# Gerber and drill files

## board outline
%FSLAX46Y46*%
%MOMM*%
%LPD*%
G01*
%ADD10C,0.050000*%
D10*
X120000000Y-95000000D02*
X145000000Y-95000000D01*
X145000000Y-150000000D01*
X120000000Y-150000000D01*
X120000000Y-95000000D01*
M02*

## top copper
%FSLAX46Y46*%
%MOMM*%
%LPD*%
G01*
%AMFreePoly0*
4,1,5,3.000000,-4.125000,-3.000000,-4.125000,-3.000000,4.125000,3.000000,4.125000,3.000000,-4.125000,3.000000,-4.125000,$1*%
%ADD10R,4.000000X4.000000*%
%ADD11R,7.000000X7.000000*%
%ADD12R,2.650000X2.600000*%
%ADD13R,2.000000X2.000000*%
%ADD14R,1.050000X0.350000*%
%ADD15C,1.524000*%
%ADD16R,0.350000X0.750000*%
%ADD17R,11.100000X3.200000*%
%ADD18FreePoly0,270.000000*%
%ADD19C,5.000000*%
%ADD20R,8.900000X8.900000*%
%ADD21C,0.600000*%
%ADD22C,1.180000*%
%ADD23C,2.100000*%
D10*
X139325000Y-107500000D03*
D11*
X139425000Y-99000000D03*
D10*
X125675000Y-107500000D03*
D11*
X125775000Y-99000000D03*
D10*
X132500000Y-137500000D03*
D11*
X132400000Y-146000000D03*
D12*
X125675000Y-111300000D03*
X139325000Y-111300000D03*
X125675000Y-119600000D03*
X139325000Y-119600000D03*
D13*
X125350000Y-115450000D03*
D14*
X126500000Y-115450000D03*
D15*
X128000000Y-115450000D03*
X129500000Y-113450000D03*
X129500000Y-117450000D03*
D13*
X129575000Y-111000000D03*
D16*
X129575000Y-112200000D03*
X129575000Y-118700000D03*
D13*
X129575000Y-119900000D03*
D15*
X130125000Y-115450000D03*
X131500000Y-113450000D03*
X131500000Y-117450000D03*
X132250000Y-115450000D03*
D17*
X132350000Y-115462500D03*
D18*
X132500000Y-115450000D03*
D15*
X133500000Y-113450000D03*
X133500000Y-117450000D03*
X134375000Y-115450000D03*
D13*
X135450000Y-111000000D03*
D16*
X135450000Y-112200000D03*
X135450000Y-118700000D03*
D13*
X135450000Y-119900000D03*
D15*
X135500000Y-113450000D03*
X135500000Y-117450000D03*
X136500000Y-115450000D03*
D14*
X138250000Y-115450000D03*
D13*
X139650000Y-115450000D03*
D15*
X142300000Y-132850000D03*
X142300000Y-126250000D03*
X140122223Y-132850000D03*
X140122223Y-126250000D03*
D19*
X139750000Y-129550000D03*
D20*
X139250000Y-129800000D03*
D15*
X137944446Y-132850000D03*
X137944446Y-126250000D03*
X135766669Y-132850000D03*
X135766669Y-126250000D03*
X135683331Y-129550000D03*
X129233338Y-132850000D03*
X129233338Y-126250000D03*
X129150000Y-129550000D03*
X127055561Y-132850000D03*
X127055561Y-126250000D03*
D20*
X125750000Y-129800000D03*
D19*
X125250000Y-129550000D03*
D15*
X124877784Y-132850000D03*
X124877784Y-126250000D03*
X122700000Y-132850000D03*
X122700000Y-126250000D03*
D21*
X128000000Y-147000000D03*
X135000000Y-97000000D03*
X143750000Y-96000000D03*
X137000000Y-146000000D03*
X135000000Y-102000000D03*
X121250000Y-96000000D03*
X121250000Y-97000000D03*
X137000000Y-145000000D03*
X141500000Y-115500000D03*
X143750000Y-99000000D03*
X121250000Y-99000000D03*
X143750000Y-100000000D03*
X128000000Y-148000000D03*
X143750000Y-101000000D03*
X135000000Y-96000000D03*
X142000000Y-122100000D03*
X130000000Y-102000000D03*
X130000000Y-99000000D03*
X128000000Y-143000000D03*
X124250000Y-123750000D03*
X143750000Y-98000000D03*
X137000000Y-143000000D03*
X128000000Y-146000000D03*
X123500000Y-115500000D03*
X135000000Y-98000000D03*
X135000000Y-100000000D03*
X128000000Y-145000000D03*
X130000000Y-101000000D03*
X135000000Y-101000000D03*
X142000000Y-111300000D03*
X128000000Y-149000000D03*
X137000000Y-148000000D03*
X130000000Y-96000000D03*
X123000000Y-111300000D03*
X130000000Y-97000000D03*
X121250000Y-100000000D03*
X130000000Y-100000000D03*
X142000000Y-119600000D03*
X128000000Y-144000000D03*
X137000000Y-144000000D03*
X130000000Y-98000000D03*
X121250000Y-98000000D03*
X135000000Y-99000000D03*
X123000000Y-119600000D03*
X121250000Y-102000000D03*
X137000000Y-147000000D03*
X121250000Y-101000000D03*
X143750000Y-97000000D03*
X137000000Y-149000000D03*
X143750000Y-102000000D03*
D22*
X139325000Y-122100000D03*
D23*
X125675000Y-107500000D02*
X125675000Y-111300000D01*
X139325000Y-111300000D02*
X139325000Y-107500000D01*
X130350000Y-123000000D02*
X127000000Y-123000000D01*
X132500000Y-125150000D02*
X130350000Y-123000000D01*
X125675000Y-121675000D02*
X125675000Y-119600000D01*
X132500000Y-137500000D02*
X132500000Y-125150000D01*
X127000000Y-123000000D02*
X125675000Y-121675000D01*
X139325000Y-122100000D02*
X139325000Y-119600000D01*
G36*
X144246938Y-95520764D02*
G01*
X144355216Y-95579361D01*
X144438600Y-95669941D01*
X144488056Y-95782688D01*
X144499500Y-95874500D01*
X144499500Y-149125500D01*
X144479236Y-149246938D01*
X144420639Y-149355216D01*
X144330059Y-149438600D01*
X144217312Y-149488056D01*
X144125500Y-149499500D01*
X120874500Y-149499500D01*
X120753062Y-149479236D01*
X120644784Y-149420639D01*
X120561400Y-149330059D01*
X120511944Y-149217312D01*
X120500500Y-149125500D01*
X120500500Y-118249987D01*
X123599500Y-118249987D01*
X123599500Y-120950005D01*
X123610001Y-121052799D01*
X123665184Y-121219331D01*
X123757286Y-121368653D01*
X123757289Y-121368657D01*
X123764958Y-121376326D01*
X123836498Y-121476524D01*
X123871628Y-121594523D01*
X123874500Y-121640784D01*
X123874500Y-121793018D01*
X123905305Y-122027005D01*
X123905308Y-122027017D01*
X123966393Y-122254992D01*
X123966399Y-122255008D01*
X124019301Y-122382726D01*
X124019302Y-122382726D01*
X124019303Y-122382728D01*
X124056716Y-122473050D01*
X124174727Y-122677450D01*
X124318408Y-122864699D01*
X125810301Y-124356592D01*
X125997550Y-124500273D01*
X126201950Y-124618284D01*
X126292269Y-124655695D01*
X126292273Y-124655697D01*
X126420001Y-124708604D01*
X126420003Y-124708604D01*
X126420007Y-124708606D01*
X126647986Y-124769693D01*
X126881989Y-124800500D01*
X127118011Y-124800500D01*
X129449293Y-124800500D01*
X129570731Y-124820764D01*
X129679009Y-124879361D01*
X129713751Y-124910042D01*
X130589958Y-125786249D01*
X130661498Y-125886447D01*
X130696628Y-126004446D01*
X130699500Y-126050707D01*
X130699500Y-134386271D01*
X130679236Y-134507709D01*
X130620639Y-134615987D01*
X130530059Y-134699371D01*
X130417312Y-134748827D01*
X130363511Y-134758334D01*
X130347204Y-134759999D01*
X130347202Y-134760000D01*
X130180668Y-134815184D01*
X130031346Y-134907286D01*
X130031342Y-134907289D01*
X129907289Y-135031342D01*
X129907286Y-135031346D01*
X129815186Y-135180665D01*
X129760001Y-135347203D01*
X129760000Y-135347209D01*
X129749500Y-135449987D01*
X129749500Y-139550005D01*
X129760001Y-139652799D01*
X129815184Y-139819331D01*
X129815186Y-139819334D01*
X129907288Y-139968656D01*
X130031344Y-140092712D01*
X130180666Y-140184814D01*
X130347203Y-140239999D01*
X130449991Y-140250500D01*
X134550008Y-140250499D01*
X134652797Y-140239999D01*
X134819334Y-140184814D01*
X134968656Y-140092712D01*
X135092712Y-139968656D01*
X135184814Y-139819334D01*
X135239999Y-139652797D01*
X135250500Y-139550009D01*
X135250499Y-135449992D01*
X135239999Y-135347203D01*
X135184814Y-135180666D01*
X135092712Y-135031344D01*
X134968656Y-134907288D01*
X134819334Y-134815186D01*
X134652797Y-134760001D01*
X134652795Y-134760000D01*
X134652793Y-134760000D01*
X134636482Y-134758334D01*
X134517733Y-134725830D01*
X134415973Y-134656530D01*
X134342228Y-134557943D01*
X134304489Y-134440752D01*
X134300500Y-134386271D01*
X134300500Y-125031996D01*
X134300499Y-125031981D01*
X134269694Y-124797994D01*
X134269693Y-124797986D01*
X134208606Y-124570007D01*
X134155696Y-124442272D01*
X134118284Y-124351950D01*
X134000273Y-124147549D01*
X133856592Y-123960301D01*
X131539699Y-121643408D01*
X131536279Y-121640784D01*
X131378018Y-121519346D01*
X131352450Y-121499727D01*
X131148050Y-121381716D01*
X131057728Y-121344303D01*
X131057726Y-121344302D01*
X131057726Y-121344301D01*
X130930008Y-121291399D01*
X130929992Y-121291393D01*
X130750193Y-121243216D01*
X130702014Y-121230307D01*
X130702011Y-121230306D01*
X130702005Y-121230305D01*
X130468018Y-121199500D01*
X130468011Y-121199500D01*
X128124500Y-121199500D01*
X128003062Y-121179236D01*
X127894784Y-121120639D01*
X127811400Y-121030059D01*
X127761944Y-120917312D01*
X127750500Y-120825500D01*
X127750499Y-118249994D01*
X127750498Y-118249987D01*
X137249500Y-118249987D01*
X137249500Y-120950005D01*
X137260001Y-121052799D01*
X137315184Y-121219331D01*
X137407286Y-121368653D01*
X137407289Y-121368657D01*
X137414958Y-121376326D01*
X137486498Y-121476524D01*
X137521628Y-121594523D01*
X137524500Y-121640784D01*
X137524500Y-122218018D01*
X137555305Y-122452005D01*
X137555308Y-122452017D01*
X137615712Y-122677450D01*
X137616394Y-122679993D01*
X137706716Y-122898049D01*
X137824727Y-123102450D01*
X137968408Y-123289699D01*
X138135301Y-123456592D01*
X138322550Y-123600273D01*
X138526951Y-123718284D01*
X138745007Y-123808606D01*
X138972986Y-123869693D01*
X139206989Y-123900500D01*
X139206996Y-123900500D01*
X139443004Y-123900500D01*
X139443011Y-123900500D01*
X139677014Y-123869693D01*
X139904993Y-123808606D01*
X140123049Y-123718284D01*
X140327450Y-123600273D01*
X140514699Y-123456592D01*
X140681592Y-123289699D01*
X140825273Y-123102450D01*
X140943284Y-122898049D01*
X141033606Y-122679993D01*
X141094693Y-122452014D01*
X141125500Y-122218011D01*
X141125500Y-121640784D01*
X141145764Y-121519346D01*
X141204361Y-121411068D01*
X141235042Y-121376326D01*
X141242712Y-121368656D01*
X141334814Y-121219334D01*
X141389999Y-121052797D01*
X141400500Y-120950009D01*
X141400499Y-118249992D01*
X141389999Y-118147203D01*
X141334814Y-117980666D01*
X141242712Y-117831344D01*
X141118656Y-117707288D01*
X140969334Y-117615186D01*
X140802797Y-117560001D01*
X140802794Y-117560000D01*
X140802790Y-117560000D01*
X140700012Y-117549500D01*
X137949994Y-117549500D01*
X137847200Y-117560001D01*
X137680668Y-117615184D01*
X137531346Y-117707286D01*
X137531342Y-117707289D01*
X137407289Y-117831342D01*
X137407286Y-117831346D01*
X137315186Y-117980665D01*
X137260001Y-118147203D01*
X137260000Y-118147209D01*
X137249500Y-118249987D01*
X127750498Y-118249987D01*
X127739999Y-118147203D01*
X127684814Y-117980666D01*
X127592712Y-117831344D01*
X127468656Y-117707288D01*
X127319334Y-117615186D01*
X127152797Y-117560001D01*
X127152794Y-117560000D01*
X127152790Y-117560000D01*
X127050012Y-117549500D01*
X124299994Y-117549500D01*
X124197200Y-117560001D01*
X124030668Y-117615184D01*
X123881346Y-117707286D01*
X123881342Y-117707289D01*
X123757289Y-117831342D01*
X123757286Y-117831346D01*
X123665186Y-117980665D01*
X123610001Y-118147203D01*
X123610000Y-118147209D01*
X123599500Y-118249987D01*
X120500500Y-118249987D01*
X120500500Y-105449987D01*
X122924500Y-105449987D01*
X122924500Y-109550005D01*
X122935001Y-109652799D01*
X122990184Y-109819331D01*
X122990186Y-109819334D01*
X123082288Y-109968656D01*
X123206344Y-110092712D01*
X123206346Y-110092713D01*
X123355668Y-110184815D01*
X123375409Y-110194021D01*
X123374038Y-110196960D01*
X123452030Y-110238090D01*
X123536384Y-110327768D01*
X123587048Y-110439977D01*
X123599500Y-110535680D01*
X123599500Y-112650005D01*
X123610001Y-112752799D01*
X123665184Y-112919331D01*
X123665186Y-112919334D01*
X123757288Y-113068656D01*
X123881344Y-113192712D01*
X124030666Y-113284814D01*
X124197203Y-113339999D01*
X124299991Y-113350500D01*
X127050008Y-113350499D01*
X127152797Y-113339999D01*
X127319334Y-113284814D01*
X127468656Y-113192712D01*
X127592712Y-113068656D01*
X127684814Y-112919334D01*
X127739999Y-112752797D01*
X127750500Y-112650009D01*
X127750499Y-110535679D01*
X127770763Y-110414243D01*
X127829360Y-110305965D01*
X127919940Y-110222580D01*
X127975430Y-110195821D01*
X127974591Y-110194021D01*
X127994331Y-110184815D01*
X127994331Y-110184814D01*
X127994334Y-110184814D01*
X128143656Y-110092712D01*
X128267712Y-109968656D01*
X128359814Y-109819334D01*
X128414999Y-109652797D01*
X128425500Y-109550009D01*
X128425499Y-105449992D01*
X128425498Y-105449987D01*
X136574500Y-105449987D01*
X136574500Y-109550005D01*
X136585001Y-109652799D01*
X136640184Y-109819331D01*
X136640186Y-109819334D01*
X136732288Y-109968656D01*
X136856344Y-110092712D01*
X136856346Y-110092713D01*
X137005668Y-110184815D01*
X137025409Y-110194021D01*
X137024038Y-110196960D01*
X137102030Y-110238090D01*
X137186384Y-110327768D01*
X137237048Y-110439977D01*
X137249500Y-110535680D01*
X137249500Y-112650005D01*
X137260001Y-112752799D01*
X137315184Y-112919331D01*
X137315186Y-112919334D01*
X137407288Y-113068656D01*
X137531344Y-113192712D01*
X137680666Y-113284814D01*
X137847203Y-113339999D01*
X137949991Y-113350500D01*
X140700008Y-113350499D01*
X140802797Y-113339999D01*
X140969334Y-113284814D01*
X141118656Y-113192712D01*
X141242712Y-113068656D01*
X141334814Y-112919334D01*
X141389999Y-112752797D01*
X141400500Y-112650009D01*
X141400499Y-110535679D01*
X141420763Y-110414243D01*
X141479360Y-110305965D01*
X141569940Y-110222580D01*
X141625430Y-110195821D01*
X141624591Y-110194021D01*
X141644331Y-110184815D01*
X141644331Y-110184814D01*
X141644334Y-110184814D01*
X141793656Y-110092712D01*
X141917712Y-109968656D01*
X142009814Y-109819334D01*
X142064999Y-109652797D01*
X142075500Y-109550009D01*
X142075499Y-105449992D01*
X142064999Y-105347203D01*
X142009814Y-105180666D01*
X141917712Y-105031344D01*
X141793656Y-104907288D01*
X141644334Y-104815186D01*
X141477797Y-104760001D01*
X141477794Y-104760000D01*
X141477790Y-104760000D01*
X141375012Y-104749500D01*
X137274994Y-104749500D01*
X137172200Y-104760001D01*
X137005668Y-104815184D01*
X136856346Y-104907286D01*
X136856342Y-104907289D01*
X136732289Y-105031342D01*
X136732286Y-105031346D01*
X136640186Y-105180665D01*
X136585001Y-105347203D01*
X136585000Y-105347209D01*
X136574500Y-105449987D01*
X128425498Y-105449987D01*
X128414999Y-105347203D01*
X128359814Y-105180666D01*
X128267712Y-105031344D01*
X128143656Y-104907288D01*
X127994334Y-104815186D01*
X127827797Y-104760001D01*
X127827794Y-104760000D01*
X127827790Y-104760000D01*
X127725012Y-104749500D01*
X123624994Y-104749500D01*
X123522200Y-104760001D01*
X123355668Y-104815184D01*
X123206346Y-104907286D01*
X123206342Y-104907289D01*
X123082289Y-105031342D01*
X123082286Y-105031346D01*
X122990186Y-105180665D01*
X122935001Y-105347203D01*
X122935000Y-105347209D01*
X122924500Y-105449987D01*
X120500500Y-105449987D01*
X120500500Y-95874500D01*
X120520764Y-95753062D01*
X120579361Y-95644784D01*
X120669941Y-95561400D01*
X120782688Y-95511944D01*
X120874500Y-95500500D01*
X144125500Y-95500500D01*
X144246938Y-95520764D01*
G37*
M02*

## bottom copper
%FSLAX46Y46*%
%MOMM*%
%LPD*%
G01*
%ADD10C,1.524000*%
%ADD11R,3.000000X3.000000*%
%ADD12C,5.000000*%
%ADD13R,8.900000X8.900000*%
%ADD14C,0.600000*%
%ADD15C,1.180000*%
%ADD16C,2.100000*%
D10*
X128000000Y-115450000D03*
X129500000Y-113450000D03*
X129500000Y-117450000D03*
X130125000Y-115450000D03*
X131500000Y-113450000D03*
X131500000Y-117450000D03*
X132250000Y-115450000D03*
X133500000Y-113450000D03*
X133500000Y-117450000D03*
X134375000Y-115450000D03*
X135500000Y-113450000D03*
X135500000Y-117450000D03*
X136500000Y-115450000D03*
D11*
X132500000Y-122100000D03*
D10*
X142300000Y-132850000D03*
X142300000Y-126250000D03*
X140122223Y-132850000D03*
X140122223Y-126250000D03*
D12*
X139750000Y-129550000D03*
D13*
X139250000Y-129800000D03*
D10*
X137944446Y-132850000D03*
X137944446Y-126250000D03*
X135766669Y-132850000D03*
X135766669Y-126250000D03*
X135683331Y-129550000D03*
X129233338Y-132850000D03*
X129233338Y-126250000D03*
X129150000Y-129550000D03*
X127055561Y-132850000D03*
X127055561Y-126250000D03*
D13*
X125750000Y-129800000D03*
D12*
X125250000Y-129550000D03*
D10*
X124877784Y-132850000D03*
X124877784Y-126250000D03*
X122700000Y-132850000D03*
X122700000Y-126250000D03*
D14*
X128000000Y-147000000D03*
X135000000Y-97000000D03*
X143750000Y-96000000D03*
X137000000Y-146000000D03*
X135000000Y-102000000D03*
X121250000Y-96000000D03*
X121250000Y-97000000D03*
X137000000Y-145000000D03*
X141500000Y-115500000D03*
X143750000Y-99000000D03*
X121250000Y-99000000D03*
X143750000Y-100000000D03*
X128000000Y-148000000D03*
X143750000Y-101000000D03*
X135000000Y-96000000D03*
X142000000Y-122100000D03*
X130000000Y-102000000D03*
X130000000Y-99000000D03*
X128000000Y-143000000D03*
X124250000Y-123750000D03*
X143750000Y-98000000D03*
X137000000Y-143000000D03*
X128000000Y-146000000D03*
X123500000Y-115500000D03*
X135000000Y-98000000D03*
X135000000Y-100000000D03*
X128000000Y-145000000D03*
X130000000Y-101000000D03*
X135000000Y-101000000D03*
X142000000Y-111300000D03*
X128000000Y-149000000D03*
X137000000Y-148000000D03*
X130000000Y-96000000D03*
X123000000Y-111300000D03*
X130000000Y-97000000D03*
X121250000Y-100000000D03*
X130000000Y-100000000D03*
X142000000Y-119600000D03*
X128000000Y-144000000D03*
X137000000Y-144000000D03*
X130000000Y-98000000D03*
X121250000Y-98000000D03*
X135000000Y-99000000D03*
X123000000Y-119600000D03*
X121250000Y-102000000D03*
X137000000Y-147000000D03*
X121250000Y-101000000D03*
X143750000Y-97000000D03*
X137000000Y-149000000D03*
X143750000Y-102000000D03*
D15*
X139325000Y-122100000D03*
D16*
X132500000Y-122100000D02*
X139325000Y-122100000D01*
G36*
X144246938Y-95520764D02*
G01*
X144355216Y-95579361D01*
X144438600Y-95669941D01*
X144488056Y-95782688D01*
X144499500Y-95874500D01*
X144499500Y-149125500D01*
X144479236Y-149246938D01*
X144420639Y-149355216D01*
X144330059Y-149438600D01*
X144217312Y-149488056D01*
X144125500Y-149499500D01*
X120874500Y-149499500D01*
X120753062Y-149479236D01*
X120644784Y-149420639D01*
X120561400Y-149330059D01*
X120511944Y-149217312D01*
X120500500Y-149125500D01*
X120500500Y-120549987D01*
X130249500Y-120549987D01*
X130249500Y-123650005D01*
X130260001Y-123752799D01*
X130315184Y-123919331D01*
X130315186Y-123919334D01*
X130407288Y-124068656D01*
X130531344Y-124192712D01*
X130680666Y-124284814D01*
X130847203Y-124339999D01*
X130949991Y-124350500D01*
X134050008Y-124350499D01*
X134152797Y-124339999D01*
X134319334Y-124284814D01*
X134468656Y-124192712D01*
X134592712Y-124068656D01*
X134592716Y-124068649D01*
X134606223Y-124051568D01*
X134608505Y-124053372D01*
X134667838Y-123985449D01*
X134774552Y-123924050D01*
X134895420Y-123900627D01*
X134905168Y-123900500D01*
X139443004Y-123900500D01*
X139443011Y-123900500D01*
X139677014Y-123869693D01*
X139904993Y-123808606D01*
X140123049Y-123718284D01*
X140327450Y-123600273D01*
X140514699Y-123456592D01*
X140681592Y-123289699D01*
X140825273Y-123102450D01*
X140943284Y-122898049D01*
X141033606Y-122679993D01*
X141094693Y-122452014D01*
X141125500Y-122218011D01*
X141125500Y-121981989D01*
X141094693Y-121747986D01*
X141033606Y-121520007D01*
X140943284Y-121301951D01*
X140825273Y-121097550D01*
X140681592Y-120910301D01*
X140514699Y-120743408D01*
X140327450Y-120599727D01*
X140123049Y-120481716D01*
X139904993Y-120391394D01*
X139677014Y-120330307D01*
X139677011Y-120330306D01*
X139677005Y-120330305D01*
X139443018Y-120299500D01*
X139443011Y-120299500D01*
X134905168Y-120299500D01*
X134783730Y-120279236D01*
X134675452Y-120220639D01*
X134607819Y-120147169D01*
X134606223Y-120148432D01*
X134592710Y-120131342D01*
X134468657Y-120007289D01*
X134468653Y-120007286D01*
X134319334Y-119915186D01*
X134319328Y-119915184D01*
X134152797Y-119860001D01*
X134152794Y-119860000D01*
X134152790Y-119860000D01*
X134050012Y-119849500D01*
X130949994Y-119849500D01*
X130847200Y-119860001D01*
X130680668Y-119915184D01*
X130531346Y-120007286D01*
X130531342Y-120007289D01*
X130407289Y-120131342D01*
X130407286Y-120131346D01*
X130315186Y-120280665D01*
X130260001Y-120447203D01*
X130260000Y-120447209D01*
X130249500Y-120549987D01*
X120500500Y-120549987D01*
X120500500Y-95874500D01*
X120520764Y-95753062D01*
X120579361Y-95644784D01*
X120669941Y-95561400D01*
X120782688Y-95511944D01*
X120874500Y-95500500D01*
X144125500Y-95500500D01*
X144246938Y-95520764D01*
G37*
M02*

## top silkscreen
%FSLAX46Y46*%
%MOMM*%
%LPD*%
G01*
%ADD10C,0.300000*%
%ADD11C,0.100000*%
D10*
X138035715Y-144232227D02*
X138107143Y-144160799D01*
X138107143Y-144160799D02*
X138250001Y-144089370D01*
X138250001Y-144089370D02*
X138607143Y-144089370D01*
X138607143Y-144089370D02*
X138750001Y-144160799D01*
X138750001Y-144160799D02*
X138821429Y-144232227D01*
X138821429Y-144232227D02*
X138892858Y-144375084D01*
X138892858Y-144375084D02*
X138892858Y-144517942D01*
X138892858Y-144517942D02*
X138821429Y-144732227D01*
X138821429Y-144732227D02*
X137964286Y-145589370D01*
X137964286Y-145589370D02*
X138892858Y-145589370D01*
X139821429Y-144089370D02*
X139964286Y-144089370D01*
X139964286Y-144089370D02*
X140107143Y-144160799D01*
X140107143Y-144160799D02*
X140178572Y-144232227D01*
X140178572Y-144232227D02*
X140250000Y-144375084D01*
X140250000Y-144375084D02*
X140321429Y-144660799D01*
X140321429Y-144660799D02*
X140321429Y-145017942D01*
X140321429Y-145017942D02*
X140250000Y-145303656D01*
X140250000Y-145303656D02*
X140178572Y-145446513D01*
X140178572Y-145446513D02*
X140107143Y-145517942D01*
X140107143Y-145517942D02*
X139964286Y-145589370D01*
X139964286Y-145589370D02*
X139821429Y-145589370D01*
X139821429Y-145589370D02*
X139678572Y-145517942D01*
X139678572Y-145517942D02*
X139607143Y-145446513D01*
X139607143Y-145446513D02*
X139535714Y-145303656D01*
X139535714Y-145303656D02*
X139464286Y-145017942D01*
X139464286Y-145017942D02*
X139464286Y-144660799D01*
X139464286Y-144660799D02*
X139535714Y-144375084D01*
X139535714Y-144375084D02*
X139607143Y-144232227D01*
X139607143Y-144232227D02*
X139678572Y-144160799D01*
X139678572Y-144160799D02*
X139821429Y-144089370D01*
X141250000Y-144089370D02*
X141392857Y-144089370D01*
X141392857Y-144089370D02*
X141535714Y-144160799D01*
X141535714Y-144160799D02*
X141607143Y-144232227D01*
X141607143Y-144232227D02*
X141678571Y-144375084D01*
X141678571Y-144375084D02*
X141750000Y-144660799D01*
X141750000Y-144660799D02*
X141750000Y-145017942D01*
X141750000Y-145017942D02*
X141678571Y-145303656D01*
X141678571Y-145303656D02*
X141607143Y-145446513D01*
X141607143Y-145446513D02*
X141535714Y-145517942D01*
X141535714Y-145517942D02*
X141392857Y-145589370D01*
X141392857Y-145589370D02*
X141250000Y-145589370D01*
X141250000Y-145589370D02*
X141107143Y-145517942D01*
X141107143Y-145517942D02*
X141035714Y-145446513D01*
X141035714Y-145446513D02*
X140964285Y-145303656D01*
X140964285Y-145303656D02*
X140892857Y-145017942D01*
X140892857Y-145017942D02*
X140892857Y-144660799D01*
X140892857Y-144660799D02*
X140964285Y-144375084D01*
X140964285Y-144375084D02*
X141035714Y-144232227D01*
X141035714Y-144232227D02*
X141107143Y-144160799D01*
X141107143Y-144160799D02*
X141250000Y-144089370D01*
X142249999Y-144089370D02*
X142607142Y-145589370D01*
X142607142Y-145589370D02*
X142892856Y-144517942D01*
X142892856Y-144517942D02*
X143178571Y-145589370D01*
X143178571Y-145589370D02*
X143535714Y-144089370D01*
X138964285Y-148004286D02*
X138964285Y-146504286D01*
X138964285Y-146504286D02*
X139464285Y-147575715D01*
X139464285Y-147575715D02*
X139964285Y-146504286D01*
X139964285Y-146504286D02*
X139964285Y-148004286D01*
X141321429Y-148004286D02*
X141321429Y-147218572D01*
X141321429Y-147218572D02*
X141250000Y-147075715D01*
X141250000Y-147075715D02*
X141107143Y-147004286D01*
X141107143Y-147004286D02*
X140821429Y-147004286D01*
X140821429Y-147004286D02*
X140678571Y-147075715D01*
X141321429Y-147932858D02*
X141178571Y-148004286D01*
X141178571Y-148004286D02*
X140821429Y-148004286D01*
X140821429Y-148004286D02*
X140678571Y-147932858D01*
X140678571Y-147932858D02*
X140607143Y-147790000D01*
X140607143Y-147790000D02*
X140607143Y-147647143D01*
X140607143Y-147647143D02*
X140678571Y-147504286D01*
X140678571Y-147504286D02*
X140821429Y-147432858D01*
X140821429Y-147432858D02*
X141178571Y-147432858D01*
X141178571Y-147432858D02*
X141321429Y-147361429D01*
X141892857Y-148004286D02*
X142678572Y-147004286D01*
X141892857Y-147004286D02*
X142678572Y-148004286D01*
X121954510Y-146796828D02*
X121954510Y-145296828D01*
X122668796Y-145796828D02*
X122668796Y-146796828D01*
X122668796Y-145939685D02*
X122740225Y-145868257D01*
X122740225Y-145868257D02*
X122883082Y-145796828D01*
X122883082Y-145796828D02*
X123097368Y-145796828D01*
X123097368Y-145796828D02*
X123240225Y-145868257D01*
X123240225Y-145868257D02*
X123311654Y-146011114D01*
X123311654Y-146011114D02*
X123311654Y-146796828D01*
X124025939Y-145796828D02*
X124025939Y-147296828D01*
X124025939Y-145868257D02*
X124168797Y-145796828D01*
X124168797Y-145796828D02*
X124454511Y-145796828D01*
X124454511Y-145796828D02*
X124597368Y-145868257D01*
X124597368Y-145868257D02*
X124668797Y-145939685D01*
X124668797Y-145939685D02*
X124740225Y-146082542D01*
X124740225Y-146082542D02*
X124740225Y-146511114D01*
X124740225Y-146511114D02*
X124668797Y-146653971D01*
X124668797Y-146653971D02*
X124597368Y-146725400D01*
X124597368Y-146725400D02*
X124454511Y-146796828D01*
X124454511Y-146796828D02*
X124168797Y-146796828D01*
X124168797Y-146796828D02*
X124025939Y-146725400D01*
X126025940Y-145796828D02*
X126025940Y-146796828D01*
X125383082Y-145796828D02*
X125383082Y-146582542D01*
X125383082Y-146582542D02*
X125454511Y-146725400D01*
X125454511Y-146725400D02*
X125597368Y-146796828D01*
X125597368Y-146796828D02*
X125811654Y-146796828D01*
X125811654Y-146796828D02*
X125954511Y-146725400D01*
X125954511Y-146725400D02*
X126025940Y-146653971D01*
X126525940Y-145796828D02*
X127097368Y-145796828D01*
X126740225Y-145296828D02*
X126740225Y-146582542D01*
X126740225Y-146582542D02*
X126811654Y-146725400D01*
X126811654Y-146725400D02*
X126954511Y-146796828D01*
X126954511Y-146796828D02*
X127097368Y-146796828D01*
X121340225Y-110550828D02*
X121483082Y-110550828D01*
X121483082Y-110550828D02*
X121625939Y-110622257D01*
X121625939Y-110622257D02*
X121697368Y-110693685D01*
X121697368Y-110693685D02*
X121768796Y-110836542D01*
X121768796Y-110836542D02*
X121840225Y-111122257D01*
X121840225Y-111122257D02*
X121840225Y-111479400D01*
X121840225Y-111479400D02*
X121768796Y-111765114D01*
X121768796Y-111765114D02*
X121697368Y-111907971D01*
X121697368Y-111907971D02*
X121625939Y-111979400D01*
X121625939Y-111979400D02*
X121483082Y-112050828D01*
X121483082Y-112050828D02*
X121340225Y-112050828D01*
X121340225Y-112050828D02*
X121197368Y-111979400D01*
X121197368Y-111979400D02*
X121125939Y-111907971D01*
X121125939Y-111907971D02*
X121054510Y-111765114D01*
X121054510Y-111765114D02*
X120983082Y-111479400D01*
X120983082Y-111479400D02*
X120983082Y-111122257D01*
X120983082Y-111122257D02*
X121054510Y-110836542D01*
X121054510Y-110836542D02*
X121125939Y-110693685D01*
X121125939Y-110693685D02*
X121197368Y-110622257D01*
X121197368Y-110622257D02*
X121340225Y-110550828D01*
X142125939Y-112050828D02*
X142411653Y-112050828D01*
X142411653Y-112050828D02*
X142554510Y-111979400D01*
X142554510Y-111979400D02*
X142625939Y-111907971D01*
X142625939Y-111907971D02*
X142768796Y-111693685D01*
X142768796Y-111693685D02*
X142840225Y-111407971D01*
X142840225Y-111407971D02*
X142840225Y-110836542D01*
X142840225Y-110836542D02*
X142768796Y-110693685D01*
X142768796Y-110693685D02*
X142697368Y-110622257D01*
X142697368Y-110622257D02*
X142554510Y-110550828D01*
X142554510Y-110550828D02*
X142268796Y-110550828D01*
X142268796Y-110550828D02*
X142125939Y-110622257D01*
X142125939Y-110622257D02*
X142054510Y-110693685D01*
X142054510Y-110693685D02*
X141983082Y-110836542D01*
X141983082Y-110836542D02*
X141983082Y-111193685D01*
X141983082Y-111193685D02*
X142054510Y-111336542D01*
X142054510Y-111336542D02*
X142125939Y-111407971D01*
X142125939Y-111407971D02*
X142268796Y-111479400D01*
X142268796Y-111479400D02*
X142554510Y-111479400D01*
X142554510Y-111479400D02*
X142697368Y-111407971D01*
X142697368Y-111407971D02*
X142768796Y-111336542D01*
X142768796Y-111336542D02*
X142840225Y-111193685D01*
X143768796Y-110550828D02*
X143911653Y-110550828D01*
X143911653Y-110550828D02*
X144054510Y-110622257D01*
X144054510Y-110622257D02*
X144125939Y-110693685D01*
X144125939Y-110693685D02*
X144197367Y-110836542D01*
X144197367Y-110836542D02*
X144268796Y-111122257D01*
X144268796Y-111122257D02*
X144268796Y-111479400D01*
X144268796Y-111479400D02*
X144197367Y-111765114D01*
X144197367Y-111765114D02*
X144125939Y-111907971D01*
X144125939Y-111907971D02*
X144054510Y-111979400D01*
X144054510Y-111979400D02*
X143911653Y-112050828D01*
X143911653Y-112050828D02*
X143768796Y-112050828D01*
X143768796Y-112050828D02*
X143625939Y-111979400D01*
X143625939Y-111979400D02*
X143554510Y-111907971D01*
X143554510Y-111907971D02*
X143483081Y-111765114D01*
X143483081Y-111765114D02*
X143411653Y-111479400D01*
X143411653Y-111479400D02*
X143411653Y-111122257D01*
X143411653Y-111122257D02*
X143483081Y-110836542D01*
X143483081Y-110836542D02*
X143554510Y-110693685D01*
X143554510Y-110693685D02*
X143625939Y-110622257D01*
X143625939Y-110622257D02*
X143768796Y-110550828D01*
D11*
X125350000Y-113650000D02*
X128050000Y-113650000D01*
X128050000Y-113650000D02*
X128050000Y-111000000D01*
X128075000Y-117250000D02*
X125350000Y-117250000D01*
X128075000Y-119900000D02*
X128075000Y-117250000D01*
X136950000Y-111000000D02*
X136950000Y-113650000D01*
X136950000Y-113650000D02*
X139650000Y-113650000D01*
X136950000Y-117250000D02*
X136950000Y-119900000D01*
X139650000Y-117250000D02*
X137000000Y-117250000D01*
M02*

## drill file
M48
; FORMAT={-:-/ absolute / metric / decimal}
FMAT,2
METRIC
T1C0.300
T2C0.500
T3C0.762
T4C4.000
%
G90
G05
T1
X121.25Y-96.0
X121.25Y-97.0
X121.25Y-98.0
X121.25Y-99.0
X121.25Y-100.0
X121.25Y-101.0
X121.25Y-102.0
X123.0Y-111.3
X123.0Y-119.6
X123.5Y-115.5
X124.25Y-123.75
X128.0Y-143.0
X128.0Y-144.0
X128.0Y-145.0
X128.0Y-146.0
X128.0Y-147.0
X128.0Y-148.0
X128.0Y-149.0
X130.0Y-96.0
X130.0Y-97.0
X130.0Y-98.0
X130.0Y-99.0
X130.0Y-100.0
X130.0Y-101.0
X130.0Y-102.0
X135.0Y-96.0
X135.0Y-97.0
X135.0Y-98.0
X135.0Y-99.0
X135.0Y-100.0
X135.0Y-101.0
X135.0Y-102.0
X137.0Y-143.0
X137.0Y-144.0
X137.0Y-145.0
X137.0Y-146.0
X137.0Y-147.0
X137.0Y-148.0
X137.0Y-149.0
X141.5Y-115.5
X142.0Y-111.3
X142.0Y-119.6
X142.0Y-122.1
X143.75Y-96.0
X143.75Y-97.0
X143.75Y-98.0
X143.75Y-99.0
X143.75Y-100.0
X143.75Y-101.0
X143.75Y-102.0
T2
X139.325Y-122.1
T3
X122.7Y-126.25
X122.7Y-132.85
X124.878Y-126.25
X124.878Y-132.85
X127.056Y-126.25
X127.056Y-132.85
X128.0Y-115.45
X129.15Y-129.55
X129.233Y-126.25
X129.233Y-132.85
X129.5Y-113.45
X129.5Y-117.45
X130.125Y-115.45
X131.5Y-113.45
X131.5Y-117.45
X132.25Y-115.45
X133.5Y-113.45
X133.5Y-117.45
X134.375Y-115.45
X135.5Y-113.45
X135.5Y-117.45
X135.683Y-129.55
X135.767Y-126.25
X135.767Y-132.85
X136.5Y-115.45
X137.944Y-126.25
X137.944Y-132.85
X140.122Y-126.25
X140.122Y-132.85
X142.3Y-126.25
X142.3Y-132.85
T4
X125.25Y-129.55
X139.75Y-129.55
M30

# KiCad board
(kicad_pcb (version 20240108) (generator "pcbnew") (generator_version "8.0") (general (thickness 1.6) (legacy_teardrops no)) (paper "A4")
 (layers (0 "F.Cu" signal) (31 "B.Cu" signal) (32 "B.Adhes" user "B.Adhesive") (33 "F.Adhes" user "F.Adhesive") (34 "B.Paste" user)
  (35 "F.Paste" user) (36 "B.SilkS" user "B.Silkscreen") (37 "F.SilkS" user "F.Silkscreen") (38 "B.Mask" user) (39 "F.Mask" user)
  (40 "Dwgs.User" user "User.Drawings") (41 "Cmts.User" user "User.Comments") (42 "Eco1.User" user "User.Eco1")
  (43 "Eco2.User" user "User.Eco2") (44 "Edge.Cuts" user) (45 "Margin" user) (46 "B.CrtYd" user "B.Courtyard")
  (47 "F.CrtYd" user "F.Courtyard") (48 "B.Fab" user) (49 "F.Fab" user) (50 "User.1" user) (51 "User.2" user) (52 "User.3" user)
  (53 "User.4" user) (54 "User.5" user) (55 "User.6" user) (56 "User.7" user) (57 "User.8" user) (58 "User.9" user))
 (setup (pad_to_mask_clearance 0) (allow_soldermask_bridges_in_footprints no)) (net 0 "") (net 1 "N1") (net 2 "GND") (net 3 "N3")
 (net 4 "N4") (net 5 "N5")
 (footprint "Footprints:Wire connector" (layer "F.Cu") (at 139.325 103.5 90)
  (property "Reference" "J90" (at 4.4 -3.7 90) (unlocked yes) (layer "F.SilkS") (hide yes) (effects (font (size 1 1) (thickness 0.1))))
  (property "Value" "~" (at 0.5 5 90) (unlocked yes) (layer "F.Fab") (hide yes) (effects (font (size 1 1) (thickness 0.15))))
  (pad "1" smd rect (at -4 0) (size 4 4) (layers "F.Cu" "F.Paste" "F.Mask") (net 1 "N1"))
  (pad "2" smd rect (at 4.5 0.1) (size 7 7) (layers "F.Cu" "F.Paste" "F.Mask") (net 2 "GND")))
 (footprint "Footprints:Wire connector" (layer "F.Cu") (at 125.675 103.5 90)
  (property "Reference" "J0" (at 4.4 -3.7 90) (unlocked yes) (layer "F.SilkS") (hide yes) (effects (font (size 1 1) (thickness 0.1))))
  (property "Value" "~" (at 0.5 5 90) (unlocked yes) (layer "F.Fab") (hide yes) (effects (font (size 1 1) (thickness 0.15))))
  (pad "1" smd rect (at -4 0) (size 4 4) (layers "F.Cu" "F.Paste" "F.Mask") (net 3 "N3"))
  (pad "2" smd rect (at 4.5 0.1) (size 7 7) (layers "F.Cu" "F.Paste" "F.Mask") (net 2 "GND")))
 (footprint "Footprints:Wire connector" (layer "F.Cu") (at 132.5 141.5 -90)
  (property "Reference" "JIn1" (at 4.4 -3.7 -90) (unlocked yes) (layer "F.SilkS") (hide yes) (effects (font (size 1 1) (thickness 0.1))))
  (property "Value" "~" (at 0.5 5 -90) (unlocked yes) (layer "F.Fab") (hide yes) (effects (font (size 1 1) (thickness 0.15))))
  (pad "1" smd rect (at -4 0 180) (size 4 4) (layers "F.Cu" "F.Paste" "F.Mask") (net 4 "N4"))
  (pad "2" smd rect (at 4.5 0.1 180) (size 7 7) (layers "F.Cu" "F.Paste" "F.Mask") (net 2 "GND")))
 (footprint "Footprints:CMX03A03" (layer "F.Cu") (at 132.5 115.45)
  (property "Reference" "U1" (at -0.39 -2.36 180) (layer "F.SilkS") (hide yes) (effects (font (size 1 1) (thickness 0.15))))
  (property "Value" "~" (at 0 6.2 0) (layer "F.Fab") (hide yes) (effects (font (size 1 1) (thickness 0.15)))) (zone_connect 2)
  (fp_line (start -7.15 -1.8) (end -4.45 -1.8) (stroke (width 0.1) (type default)) (layer "F.SilkS"))
  (fp_line (start -4.45 -1.8) (end -4.45 -4.45) (stroke (width 0.1) (type default)) (layer "F.SilkS"))
  (fp_line (start -4.425 1.8) (end -7.15 1.8) (stroke (width 0.1) (type default)) (layer "F.SilkS"))
  (fp_line (start -4.425 4.45) (end -4.425 1.8) (stroke (width 0.1) (type default)) (layer "F.SilkS"))
  (fp_line (start 4.45 -4.45) (end 4.45 -1.8) (stroke (width 0.1) (type default)) (layer "F.SilkS"))
  (fp_line (start 4.45 -1.8) (end 7.15 -1.8) (stroke (width 0.1) (type default)) (layer "F.SilkS"))
  (fp_line (start 4.45 1.8) (end 4.45 4.45) (stroke (width 0.1) (type default)) (layer "F.SilkS"))
  (fp_line (start 7.15 1.8) (end 4.5 1.8) (stroke (width 0.1) (type default)) (layer "F.SilkS"))
  (pad "1" smd rect (at -6.825 -4.15 270) (size 2.6 2.65) (layers "F.Cu" "F.Paste" "F.Mask") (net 3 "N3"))
  (pad "2" smd rect (at 6.825 -4.15 270) (size 2.6 2.65) (layers "F.Cu" "F.Paste" "F.Mask") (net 1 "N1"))
  (pad "3" smd rect (at -6.825 4.15 270) (size 2.6 2.65) (layers "F.Cu" "F.Paste" "F.Mask") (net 4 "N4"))
  (pad "4" smd rect (at 6.825 4.15 270) (size 2.6 2.65) (layers "F.Cu" "F.Paste" "F.Mask") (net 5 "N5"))
  (pad "5" smd rect (at -7.15 0) (size 2 2) (layers "F.Cu" "F.Paste" "F.Mask") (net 2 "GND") (zone_connect 2))
  (pad "5" smd rect (at -6 0) (size 1.05 0.35) (layers "F.Cu" "F.Mask") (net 2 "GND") (zone_connect 2))
  (pad "5" thru_hole circle (at -4.5 0) (size 1.524 1.524) (drill 0.762) (layers "*.Cu" "*.Mask") (remove_unused_layers no) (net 2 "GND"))
  (pad "5" thru_hole circle (at -3 -2) (size 1.524 1.524) (drill 0.762) (layers "*.Cu" "*.Mask") (remove_unused_layers no) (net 2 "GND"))
  (pad "5" thru_hole circle (at -3 2) (size 1.524 1.524) (drill 0.762) (layers "*.Cu" "*.Mask") (remove_unused_layers no) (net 2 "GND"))
  (pad "5" smd rect (at -2.925 -4.45 270) (size 2 2) (layers "F.Cu" "F.Paste" "F.Mask") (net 2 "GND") (zone_connect 2))
  (pad "5" smd rect (at -2.925 -3.25 90) (size 0.75 0.35) (layers "F.Cu" "F.Mask") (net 2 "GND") (zone_connect 2))
  (pad "5" smd rect (at -2.925 3.25 90) (size 0.75 0.35) (layers "F.Cu" "F.Mask") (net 2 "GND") (zone_connect 2))
  (pad "5" smd rect (at -2.925 4.45 270) (size 2 2) (layers "F.Cu" "F.Paste" "F.Mask") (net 2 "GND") (zone_connect 2))
  (pad "5" thru_hole circle (at -2.375 0) (size 1.524 1.524) (drill 0.762) (layers "*.Cu" "*.Mask") (remove_unused_layers no) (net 2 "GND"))
  (pad "5" thru_hole circle (at -1 -2) (size 1.524 1.524) (drill 0.762) (layers "*.Cu" "*.Mask") (remove_unused_layers no) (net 2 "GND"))
  (pad "5" thru_hole circle (at -1 2) (size 1.524 1.524) (drill 0.762) (layers "*.Cu" "*.Mask") (remove_unused_layers no) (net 2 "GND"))
  (pad "5" thru_hole circle (at -0.25 0) (size 1.524 1.524) (drill 0.762) (layers "*.Cu" "*.Mask") (remove_unused_layers no) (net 2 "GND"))
  (pad "5" smd rect (at -0.15 0.0125) (size 11.1 3.2) (layers "F.Cu" "F.Mask") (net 2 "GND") (zone_connect 2))
  (pad "5" smd custom (at 0 0 270) (size 6 8.25) (layers "F.Cu" "F.Mask") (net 2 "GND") (zone_connect 2)
   (options (clearance outline) (anchor rect)) (primitives))
  (pad "5" thru_hole circle (at 1 -2) (size 1.524 1.524) (drill 0.762) (layers "*.Cu" "*.Mask") (remove_unused_layers no) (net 2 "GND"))
  (pad "5" thru_hole circle (at 1 2) (size 1.524 1.524) (drill 0.762) (layers "*.Cu" "*.Mask") (remove_unused_layers no) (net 2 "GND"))
  (pad "5" thru_hole circle (at 1.875 0) (size 1.524 1.524) (drill 0.762) (layers "*.Cu" "*.Mask") (remove_unused_layers no) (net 2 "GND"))
  (pad "5" smd rect (at 2.95 -4.45 270) (size 2 2) (layers "F.Cu" "F.Paste" "F.Mask") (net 2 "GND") (zone_connect 2))
  (pad "5" smd rect (at 2.95 -3.25 90) (size 0.75 0.35) (layers "F.Cu" "F.Mask") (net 2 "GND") (zone_connect 2))
  (pad "5" smd rect (at 2.95 3.25 90) (size 0.75 0.35) (layers "F.Cu" "F.Mask") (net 2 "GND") (zone_connect 2))
  (pad "5" smd rect (at 2.95 4.45 270) (size 2 2) (layers "F.Cu" "F.Paste" "F.Mask") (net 2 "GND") (zone_connect 2))
  (pad "5" thru_hole circle (at 3 -2) (size 1.524 1.524) (drill 0.762) (layers "*.Cu" "*.Mask") (remove_unused_layers no) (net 2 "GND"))
  (pad "5" thru_hole circle (at 3 2) (size 1.524 1.524) (drill 0.762) (layers "*.Cu" "*.Mask") (remove_unused_layers no) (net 2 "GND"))
  (pad "5" thru_hole circle (at 4 0) (size 1.524 1.524) (drill 0.762) (layers "*.Cu" "*.Mask") (remove_unused_layers no) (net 2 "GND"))
  (pad "5" smd rect (at 5.75 0) (size 1.05 0.35) (layers "F.Cu" "F.Mask") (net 2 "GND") (zone_connect 2))
  (pad "5" smd rect (at 7.15 0) (size 2 2) (layers "F.Cu" "F.Paste" "F.Mask") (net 2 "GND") (zone_connect 2)))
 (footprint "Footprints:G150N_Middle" (layer "B.Cu") (at 132.5 130.1 180)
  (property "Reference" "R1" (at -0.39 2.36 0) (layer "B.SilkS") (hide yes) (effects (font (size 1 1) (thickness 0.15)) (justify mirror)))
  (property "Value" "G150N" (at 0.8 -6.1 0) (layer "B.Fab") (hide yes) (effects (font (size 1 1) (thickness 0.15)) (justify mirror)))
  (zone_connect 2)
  (pad "1" smd rect (at 0 8 270) (size 3 3) (layers "B.Cu" "B.Paste" "B.Mask") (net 5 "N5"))
  (pad "2" thru_hole circle (at -9.8 -2.75 180) (size 1.524 1.524) (drill 0.762) (layers "*.Cu" "*.Mask") (remove_unused_layers no)
   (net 2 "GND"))
  (pad "2" thru_hole circle (at -9.8 3.85 180) (size 1.524 1.524) (drill 0.762) (layers "*.Cu" "*.Mask") (remove_unused_layers no)
   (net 2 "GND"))
  (pad "2" thru_hole circle (at -7.622223 -2.75 180) (size 1.524 1.524) (drill 0.762) (layers "*.Cu" "*.Mask") (remove_unused_layers no)
   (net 2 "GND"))
  (pad "2" thru_hole circle (at -7.622223 3.85 180) (size 1.524 1.524) (drill 0.762) (layers "*.Cu" "*.Mask") (remove_unused_layers no)
   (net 2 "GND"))
  (pad "2" thru_hole circle (at -7.25 0.55 270) (size 5 5) (drill 4) (layers "*.Cu" "*.Mask") (remove_unused_layers no) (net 2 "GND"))
  (pad "2" smd rect (at -6.75 0.3 270) (size 8.9 8.9) (layers "F.Cu" "F.Mask") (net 2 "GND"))
  (pad "2" smd rect (at -6.75 0.3 270) (size 8.9 8.9) (layers "B.Cu" "B.Mask") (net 2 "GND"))
  (pad "2" thru_hole circle (at -5.444446 -2.75 180) (size 1.524 1.524) (drill 0.762) (layers "*.Cu" "*.Mask") (remove_unused_layers no)
   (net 2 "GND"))
  (pad "2" thru_hole circle (at -5.444446 3.85 180) (size 1.524 1.524) (drill 0.762) (layers "*.Cu" "*.Mask") (remove_unused_layers no)
   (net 2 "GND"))
  (pad "2" thru_hole circle (at -3.266669 -2.75 180) (size 1.524 1.524) (drill 0.762) (layers "*.Cu" "*.Mask") (remove_unused_layers no)
   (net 2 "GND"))
  (pad "2" thru_hole circle (at -3.266669 3.85 180) (size 1.524 1.524) (drill 0.762) (layers "*.Cu" "*.Mask") (remove_unused_layers no)
   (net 2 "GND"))
  (pad "2" thru_hole circle (at -3.183331 0.55 180) (size 1.524 1.524) (drill 0.762) (layers "*.Cu" "*.Mask") (remove_unused_layers no)
   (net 2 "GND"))
  (pad "2" thru_hole circle (at 3.266662 -2.75 180) (size 1.524 1.524) (drill 0.762) (layers "*.Cu" "*.Mask") (remove_unused_layers no)
   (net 2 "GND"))
  (pad "2" thru_hole circle (at 3.266662 3.85 180) (size 1.524 1.524) (drill 0.762) (layers "*.Cu" "*.Mask") (remove_unused_layers no)
   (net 2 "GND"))
  (pad "2" thru_hole circle (at 3.35 0.55 180) (size 1.524 1.524) (drill 0.762) (layers "*.Cu" "*.Mask") (remove_unused_layers no)
   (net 2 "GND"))
  (pad "2" thru_hole circle (at 5.444439 -2.75 180) (size 1.524 1.524) (drill 0.762) (layers "*.Cu" "*.Mask") (remove_unused_layers no)
   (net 2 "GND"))
  (pad "2" thru_hole circle (at 5.444439 3.85 180) (size 1.524 1.524) (drill 0.762) (layers "*.Cu" "*.Mask") (remove_unused_layers no)
   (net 2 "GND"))
  (pad "2" smd rect (at 6.75 0.3 270) (size 8.9 8.9) (layers "F.Cu" "F.Mask") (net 2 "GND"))
  (pad "2" smd rect (at 6.75 0.3 270) (size 8.9 8.9) (layers "B.Cu" "B.Mask") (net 2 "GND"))
  (pad "2" thru_hole circle (at 7.25 0.55 270) (size 5 5) (drill 4) (layers "*.Cu" "*.Mask") (remove_unused_layers no) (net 2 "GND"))
  (pad "2" thru_hole circle (at 7.622216 -2.75 180) (size 1.524 1.524) (drill 0.762) (layers "*.Cu" "*.Mask") (remove_unused_layers no)
   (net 2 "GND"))
  (pad "2" thru_hole circle (at 7.622216 3.85 180) (size 1.524 1.524) (drill 0.762) (layers "*.Cu" "*.Mask") (remove_unused_layers no)
   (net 2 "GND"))
  (pad "2" thru_hole circle (at 9.8 -2.75 180) (size 1.524 1.524) (drill 0.762) (layers "*.Cu" "*.Mask") (remove_unused_layers no)
   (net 2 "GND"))
  (pad "2" thru_hole circle (at 9.8 3.85 180) (size 1.524 1.524) (drill 0.762) (layers "*.Cu" "*.Mask") (remove_unused_layers no)
   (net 2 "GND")))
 (gr_rect (start 120 95) (end 145 150) (stroke (width 0.05) (type default)) (fill none) (layer "Edge.Cuts"))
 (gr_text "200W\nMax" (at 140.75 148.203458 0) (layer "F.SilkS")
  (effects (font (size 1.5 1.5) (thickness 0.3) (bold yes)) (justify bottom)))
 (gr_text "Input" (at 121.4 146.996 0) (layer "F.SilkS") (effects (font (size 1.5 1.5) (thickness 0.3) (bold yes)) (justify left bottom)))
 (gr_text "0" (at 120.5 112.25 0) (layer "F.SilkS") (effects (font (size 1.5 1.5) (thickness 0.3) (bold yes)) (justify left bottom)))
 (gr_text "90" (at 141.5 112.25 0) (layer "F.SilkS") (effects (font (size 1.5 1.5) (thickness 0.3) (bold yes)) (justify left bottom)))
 (via (at 128 147) (size 0.6) (drill 0.3) (layers "F.Cu" "B.Cu") (free yes) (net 2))
 (via (at 135 97) (size 0.6) (drill 0.3) (layers "F.Cu" "B.Cu") (free yes) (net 2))
 (via (at 143.75 96) (size 0.6) (drill 0.3) (layers "F.Cu" "B.Cu") (free yes) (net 2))
 (via (at 137 146) (size 0.6) (drill 0.3) (layers "F.Cu" "B.Cu") (free yes) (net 2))
 (via (at 135 102) (size 0.6) (drill 0.3) (layers "F.Cu" "B.Cu") (free yes) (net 2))
 (via (at 121.25 96) (size 0.6) (drill 0.3) (layers "F.Cu" "B.Cu") (free yes) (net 2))
 (via (at 121.25 97) (size 0.6) (drill 0.3) (layers "F.Cu" "B.Cu") (free yes) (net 2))
 (via (at 137 145) (size 0.6) (drill 0.3) (layers "F.Cu" "B.Cu") (free yes) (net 2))
 (via (at 141.5 115.5) (size 0.6) (drill 0.3) (layers "F.Cu" "B.Cu") (free yes) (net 2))
 (via (at 143.75 99) (size 0.6) (drill 0.3) (layers "F.Cu" "B.Cu") (free yes) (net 2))
 (via (at 121.25 99) (size 0.6) (drill 0.3) (layers "F.Cu" "B.Cu") (free yes) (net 2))
 (via (at 143.75 100) (size 0.6) (drill 0.3) (layers "F.Cu" "B.Cu") (free yes) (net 2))
 (via (at 128 148) (size 0.6) (drill 0.3) (layers "F.Cu" "B.Cu") (free yes) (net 2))
 (via (at 143.75 101) (size 0.6) (drill 0.3) (layers "F.Cu" "B.Cu") (free yes) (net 2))
 (via (at 135 96) (size 0.6) (drill 0.3) (layers "F.Cu" "B.Cu") (free yes) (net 2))
 (via (at 142 122.1) (size 0.6) (drill 0.3) (layers "F.Cu" "B.Cu") (free yes) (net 2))
 (via (at 130 102) (size 0.6) (drill 0.3) (layers "F.Cu" "B.Cu") (free yes) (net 2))
 (via (at 130 99) (size 0.6) (drill 0.3) (layers "F.Cu" "B.Cu") (free yes) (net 2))
 (via (at 128 143) (size 0.6) (drill 0.3) (layers "F.Cu" "B.Cu") (free yes) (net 2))
 (via (at 124.25 123.75) (size 0.6) (drill 0.3) (layers "F.Cu" "B.Cu") (free yes) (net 2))
 (via (at 143.75 98) (size 0.6) (drill 0.3) (layers "F.Cu" "B.Cu") (free yes) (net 2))
 (via (at 137 143) (size 0.6) (drill 0.3) (layers "F.Cu" "B.Cu") (free yes) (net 2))
 (via (at 128 146) (size 0.6) (drill 0.3) (layers "F.Cu" "B.Cu") (free yes) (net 2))
 (via (at 123.5 115.5) (size 0.6) (drill 0.3) (layers "F.Cu" "B.Cu") (free yes) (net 2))
 (via (at 135 98) (size 0.6) (drill 0.3) (layers "F.Cu" "B.Cu") (free yes) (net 2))
 (via (at 135 100) (size 0.6) (drill 0.3) (layers "F.Cu" "B.Cu") (free yes) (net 2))
 (via (at 128 145) (size 0.6) (drill 0.3) (layers "F.Cu" "B.Cu") (free yes) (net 2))
 (via (at 130 101) (size 0.6) (drill 0.3) (layers "F.Cu" "B.Cu") (free yes) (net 2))
 (via (at 135 101) (size 0.6) (drill 0.3) (layers "F.Cu" "B.Cu") (free yes) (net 2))
 (via (at 142 111.3) (size 0.6) (drill 0.3) (layers "F.Cu" "B.Cu") (free yes) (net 2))
 (via (at 128 149) (size 0.6) (drill 0.3) (layers "F.Cu" "B.Cu") (free yes) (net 2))
 (via (at 137 148) (size 0.6) (drill 0.3) (layers "F.Cu" "B.Cu") (free yes) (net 2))
 (via (at 130 96) (size 0.6) (drill 0.3) (layers "F.Cu" "B.Cu") (free yes) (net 2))
 (via (at 123 111.3) (size 0.6) (drill 0.3) (layers "F.Cu" "B.Cu") (free yes) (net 2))
 (via (at 130 97) (size 0.6) (drill 0.3) (layers "F.Cu" "B.Cu") (free yes) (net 2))
 (via (at 121.25 100) (size 0.6) (drill 0.3) (layers "F.Cu" "B.Cu") (free yes) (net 2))
 (via (at 130 100) (size 0.6) (drill 0.3) (layers "F.Cu" "B.Cu") (free yes) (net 2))
 (via (at 142 119.6) (size 0.6) (drill 0.3) (layers "F.Cu" "B.Cu") (free yes) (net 2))
 (via (at 128 144) (size 0.6) (drill 0.3) (layers "F.Cu" "B.Cu") (free yes) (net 2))
 (via (at 137 144) (size 0.6) (drill 0.3) (layers "F.Cu" "B.Cu") (free yes) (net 2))
 (via (at 130 98) (size 0.6) (drill 0.3) (layers "F.Cu" "B.Cu") (free yes) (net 2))
 (via (at 121.25 98) (size 0.6) (drill 0.3) (layers "F.Cu" "B.Cu") (free yes) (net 2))
 (via (at 135 99) (size 0.6) (drill 0.3) (layers "F.Cu" "B.Cu") (free yes) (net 2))
 (via (at 123 119.6) (size 0.6) (drill 0.3) (layers "F.Cu" "B.Cu") (free yes) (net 2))
 (via (at 121.25 102) (size 0.6) (drill 0.3) (layers "F.Cu" "B.Cu") (free yes) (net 2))
 (via (at 137 147) (size 0.6) (drill 0.3) (layers "F.Cu" "B.Cu") (free yes) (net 2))
 (via (at 121.25 101) (size 0.6) (drill 0.3) (layers "F.Cu" "B.Cu") (free yes) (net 2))
 (via (at 143.75 97) (size 0.6) (drill 0.3) (layers "F.Cu" "B.Cu") (free yes) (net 2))
 (via (at 137 149) (size 0.6) (drill 0.3) (layers "F.Cu" "B.Cu") (free yes) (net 2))
 (via (at 143.75 102) (size 0.6) (drill 0.3) (layers "F.Cu" "B.Cu") (free yes) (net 2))
 (segment (start 125.675 107.5) (end 125.675 111.3) (width 2.1) (layer "F.Cu") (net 3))
 (segment (start 139.325 111.3) (end 139.325 107.5) (width 2.1) (layer "F.Cu") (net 1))
 (segment (start 130.35 123) (end 127 123) (width 2.1) (layer "F.Cu") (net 4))
 (segment (start 132.5 125.15) (end 130.35 123) (width 2.1) (layer "F.Cu") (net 4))
 (segment (start 125.675 121.675) (end 125.675 119.6) (width 2.1) (layer "F.Cu") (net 4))
 (segment (start 132.5 137.5) (end 132.5 125.15) (width 2.1) (layer "F.Cu") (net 4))
 (segment (start 127 123) (end 125.675 121.675) (width 2.1) (layer "F.Cu") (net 4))
 (segment (start 139.325 122.1) (end 139.325 119.6) (width 2.1) (layer "F.Cu") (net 5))
 (via (at 139.325 122.1) (size 1.18) (drill 0.5) (layers "F.Cu" "B.Cu") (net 5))
 (segment (start 132.5 122.1) (end 139.325 122.1) (width 2.1) (layer "B.Cu") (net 5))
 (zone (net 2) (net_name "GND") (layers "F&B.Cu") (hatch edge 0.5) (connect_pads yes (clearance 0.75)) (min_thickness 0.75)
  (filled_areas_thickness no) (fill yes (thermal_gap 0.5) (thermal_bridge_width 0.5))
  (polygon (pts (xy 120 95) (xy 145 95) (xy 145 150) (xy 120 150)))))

